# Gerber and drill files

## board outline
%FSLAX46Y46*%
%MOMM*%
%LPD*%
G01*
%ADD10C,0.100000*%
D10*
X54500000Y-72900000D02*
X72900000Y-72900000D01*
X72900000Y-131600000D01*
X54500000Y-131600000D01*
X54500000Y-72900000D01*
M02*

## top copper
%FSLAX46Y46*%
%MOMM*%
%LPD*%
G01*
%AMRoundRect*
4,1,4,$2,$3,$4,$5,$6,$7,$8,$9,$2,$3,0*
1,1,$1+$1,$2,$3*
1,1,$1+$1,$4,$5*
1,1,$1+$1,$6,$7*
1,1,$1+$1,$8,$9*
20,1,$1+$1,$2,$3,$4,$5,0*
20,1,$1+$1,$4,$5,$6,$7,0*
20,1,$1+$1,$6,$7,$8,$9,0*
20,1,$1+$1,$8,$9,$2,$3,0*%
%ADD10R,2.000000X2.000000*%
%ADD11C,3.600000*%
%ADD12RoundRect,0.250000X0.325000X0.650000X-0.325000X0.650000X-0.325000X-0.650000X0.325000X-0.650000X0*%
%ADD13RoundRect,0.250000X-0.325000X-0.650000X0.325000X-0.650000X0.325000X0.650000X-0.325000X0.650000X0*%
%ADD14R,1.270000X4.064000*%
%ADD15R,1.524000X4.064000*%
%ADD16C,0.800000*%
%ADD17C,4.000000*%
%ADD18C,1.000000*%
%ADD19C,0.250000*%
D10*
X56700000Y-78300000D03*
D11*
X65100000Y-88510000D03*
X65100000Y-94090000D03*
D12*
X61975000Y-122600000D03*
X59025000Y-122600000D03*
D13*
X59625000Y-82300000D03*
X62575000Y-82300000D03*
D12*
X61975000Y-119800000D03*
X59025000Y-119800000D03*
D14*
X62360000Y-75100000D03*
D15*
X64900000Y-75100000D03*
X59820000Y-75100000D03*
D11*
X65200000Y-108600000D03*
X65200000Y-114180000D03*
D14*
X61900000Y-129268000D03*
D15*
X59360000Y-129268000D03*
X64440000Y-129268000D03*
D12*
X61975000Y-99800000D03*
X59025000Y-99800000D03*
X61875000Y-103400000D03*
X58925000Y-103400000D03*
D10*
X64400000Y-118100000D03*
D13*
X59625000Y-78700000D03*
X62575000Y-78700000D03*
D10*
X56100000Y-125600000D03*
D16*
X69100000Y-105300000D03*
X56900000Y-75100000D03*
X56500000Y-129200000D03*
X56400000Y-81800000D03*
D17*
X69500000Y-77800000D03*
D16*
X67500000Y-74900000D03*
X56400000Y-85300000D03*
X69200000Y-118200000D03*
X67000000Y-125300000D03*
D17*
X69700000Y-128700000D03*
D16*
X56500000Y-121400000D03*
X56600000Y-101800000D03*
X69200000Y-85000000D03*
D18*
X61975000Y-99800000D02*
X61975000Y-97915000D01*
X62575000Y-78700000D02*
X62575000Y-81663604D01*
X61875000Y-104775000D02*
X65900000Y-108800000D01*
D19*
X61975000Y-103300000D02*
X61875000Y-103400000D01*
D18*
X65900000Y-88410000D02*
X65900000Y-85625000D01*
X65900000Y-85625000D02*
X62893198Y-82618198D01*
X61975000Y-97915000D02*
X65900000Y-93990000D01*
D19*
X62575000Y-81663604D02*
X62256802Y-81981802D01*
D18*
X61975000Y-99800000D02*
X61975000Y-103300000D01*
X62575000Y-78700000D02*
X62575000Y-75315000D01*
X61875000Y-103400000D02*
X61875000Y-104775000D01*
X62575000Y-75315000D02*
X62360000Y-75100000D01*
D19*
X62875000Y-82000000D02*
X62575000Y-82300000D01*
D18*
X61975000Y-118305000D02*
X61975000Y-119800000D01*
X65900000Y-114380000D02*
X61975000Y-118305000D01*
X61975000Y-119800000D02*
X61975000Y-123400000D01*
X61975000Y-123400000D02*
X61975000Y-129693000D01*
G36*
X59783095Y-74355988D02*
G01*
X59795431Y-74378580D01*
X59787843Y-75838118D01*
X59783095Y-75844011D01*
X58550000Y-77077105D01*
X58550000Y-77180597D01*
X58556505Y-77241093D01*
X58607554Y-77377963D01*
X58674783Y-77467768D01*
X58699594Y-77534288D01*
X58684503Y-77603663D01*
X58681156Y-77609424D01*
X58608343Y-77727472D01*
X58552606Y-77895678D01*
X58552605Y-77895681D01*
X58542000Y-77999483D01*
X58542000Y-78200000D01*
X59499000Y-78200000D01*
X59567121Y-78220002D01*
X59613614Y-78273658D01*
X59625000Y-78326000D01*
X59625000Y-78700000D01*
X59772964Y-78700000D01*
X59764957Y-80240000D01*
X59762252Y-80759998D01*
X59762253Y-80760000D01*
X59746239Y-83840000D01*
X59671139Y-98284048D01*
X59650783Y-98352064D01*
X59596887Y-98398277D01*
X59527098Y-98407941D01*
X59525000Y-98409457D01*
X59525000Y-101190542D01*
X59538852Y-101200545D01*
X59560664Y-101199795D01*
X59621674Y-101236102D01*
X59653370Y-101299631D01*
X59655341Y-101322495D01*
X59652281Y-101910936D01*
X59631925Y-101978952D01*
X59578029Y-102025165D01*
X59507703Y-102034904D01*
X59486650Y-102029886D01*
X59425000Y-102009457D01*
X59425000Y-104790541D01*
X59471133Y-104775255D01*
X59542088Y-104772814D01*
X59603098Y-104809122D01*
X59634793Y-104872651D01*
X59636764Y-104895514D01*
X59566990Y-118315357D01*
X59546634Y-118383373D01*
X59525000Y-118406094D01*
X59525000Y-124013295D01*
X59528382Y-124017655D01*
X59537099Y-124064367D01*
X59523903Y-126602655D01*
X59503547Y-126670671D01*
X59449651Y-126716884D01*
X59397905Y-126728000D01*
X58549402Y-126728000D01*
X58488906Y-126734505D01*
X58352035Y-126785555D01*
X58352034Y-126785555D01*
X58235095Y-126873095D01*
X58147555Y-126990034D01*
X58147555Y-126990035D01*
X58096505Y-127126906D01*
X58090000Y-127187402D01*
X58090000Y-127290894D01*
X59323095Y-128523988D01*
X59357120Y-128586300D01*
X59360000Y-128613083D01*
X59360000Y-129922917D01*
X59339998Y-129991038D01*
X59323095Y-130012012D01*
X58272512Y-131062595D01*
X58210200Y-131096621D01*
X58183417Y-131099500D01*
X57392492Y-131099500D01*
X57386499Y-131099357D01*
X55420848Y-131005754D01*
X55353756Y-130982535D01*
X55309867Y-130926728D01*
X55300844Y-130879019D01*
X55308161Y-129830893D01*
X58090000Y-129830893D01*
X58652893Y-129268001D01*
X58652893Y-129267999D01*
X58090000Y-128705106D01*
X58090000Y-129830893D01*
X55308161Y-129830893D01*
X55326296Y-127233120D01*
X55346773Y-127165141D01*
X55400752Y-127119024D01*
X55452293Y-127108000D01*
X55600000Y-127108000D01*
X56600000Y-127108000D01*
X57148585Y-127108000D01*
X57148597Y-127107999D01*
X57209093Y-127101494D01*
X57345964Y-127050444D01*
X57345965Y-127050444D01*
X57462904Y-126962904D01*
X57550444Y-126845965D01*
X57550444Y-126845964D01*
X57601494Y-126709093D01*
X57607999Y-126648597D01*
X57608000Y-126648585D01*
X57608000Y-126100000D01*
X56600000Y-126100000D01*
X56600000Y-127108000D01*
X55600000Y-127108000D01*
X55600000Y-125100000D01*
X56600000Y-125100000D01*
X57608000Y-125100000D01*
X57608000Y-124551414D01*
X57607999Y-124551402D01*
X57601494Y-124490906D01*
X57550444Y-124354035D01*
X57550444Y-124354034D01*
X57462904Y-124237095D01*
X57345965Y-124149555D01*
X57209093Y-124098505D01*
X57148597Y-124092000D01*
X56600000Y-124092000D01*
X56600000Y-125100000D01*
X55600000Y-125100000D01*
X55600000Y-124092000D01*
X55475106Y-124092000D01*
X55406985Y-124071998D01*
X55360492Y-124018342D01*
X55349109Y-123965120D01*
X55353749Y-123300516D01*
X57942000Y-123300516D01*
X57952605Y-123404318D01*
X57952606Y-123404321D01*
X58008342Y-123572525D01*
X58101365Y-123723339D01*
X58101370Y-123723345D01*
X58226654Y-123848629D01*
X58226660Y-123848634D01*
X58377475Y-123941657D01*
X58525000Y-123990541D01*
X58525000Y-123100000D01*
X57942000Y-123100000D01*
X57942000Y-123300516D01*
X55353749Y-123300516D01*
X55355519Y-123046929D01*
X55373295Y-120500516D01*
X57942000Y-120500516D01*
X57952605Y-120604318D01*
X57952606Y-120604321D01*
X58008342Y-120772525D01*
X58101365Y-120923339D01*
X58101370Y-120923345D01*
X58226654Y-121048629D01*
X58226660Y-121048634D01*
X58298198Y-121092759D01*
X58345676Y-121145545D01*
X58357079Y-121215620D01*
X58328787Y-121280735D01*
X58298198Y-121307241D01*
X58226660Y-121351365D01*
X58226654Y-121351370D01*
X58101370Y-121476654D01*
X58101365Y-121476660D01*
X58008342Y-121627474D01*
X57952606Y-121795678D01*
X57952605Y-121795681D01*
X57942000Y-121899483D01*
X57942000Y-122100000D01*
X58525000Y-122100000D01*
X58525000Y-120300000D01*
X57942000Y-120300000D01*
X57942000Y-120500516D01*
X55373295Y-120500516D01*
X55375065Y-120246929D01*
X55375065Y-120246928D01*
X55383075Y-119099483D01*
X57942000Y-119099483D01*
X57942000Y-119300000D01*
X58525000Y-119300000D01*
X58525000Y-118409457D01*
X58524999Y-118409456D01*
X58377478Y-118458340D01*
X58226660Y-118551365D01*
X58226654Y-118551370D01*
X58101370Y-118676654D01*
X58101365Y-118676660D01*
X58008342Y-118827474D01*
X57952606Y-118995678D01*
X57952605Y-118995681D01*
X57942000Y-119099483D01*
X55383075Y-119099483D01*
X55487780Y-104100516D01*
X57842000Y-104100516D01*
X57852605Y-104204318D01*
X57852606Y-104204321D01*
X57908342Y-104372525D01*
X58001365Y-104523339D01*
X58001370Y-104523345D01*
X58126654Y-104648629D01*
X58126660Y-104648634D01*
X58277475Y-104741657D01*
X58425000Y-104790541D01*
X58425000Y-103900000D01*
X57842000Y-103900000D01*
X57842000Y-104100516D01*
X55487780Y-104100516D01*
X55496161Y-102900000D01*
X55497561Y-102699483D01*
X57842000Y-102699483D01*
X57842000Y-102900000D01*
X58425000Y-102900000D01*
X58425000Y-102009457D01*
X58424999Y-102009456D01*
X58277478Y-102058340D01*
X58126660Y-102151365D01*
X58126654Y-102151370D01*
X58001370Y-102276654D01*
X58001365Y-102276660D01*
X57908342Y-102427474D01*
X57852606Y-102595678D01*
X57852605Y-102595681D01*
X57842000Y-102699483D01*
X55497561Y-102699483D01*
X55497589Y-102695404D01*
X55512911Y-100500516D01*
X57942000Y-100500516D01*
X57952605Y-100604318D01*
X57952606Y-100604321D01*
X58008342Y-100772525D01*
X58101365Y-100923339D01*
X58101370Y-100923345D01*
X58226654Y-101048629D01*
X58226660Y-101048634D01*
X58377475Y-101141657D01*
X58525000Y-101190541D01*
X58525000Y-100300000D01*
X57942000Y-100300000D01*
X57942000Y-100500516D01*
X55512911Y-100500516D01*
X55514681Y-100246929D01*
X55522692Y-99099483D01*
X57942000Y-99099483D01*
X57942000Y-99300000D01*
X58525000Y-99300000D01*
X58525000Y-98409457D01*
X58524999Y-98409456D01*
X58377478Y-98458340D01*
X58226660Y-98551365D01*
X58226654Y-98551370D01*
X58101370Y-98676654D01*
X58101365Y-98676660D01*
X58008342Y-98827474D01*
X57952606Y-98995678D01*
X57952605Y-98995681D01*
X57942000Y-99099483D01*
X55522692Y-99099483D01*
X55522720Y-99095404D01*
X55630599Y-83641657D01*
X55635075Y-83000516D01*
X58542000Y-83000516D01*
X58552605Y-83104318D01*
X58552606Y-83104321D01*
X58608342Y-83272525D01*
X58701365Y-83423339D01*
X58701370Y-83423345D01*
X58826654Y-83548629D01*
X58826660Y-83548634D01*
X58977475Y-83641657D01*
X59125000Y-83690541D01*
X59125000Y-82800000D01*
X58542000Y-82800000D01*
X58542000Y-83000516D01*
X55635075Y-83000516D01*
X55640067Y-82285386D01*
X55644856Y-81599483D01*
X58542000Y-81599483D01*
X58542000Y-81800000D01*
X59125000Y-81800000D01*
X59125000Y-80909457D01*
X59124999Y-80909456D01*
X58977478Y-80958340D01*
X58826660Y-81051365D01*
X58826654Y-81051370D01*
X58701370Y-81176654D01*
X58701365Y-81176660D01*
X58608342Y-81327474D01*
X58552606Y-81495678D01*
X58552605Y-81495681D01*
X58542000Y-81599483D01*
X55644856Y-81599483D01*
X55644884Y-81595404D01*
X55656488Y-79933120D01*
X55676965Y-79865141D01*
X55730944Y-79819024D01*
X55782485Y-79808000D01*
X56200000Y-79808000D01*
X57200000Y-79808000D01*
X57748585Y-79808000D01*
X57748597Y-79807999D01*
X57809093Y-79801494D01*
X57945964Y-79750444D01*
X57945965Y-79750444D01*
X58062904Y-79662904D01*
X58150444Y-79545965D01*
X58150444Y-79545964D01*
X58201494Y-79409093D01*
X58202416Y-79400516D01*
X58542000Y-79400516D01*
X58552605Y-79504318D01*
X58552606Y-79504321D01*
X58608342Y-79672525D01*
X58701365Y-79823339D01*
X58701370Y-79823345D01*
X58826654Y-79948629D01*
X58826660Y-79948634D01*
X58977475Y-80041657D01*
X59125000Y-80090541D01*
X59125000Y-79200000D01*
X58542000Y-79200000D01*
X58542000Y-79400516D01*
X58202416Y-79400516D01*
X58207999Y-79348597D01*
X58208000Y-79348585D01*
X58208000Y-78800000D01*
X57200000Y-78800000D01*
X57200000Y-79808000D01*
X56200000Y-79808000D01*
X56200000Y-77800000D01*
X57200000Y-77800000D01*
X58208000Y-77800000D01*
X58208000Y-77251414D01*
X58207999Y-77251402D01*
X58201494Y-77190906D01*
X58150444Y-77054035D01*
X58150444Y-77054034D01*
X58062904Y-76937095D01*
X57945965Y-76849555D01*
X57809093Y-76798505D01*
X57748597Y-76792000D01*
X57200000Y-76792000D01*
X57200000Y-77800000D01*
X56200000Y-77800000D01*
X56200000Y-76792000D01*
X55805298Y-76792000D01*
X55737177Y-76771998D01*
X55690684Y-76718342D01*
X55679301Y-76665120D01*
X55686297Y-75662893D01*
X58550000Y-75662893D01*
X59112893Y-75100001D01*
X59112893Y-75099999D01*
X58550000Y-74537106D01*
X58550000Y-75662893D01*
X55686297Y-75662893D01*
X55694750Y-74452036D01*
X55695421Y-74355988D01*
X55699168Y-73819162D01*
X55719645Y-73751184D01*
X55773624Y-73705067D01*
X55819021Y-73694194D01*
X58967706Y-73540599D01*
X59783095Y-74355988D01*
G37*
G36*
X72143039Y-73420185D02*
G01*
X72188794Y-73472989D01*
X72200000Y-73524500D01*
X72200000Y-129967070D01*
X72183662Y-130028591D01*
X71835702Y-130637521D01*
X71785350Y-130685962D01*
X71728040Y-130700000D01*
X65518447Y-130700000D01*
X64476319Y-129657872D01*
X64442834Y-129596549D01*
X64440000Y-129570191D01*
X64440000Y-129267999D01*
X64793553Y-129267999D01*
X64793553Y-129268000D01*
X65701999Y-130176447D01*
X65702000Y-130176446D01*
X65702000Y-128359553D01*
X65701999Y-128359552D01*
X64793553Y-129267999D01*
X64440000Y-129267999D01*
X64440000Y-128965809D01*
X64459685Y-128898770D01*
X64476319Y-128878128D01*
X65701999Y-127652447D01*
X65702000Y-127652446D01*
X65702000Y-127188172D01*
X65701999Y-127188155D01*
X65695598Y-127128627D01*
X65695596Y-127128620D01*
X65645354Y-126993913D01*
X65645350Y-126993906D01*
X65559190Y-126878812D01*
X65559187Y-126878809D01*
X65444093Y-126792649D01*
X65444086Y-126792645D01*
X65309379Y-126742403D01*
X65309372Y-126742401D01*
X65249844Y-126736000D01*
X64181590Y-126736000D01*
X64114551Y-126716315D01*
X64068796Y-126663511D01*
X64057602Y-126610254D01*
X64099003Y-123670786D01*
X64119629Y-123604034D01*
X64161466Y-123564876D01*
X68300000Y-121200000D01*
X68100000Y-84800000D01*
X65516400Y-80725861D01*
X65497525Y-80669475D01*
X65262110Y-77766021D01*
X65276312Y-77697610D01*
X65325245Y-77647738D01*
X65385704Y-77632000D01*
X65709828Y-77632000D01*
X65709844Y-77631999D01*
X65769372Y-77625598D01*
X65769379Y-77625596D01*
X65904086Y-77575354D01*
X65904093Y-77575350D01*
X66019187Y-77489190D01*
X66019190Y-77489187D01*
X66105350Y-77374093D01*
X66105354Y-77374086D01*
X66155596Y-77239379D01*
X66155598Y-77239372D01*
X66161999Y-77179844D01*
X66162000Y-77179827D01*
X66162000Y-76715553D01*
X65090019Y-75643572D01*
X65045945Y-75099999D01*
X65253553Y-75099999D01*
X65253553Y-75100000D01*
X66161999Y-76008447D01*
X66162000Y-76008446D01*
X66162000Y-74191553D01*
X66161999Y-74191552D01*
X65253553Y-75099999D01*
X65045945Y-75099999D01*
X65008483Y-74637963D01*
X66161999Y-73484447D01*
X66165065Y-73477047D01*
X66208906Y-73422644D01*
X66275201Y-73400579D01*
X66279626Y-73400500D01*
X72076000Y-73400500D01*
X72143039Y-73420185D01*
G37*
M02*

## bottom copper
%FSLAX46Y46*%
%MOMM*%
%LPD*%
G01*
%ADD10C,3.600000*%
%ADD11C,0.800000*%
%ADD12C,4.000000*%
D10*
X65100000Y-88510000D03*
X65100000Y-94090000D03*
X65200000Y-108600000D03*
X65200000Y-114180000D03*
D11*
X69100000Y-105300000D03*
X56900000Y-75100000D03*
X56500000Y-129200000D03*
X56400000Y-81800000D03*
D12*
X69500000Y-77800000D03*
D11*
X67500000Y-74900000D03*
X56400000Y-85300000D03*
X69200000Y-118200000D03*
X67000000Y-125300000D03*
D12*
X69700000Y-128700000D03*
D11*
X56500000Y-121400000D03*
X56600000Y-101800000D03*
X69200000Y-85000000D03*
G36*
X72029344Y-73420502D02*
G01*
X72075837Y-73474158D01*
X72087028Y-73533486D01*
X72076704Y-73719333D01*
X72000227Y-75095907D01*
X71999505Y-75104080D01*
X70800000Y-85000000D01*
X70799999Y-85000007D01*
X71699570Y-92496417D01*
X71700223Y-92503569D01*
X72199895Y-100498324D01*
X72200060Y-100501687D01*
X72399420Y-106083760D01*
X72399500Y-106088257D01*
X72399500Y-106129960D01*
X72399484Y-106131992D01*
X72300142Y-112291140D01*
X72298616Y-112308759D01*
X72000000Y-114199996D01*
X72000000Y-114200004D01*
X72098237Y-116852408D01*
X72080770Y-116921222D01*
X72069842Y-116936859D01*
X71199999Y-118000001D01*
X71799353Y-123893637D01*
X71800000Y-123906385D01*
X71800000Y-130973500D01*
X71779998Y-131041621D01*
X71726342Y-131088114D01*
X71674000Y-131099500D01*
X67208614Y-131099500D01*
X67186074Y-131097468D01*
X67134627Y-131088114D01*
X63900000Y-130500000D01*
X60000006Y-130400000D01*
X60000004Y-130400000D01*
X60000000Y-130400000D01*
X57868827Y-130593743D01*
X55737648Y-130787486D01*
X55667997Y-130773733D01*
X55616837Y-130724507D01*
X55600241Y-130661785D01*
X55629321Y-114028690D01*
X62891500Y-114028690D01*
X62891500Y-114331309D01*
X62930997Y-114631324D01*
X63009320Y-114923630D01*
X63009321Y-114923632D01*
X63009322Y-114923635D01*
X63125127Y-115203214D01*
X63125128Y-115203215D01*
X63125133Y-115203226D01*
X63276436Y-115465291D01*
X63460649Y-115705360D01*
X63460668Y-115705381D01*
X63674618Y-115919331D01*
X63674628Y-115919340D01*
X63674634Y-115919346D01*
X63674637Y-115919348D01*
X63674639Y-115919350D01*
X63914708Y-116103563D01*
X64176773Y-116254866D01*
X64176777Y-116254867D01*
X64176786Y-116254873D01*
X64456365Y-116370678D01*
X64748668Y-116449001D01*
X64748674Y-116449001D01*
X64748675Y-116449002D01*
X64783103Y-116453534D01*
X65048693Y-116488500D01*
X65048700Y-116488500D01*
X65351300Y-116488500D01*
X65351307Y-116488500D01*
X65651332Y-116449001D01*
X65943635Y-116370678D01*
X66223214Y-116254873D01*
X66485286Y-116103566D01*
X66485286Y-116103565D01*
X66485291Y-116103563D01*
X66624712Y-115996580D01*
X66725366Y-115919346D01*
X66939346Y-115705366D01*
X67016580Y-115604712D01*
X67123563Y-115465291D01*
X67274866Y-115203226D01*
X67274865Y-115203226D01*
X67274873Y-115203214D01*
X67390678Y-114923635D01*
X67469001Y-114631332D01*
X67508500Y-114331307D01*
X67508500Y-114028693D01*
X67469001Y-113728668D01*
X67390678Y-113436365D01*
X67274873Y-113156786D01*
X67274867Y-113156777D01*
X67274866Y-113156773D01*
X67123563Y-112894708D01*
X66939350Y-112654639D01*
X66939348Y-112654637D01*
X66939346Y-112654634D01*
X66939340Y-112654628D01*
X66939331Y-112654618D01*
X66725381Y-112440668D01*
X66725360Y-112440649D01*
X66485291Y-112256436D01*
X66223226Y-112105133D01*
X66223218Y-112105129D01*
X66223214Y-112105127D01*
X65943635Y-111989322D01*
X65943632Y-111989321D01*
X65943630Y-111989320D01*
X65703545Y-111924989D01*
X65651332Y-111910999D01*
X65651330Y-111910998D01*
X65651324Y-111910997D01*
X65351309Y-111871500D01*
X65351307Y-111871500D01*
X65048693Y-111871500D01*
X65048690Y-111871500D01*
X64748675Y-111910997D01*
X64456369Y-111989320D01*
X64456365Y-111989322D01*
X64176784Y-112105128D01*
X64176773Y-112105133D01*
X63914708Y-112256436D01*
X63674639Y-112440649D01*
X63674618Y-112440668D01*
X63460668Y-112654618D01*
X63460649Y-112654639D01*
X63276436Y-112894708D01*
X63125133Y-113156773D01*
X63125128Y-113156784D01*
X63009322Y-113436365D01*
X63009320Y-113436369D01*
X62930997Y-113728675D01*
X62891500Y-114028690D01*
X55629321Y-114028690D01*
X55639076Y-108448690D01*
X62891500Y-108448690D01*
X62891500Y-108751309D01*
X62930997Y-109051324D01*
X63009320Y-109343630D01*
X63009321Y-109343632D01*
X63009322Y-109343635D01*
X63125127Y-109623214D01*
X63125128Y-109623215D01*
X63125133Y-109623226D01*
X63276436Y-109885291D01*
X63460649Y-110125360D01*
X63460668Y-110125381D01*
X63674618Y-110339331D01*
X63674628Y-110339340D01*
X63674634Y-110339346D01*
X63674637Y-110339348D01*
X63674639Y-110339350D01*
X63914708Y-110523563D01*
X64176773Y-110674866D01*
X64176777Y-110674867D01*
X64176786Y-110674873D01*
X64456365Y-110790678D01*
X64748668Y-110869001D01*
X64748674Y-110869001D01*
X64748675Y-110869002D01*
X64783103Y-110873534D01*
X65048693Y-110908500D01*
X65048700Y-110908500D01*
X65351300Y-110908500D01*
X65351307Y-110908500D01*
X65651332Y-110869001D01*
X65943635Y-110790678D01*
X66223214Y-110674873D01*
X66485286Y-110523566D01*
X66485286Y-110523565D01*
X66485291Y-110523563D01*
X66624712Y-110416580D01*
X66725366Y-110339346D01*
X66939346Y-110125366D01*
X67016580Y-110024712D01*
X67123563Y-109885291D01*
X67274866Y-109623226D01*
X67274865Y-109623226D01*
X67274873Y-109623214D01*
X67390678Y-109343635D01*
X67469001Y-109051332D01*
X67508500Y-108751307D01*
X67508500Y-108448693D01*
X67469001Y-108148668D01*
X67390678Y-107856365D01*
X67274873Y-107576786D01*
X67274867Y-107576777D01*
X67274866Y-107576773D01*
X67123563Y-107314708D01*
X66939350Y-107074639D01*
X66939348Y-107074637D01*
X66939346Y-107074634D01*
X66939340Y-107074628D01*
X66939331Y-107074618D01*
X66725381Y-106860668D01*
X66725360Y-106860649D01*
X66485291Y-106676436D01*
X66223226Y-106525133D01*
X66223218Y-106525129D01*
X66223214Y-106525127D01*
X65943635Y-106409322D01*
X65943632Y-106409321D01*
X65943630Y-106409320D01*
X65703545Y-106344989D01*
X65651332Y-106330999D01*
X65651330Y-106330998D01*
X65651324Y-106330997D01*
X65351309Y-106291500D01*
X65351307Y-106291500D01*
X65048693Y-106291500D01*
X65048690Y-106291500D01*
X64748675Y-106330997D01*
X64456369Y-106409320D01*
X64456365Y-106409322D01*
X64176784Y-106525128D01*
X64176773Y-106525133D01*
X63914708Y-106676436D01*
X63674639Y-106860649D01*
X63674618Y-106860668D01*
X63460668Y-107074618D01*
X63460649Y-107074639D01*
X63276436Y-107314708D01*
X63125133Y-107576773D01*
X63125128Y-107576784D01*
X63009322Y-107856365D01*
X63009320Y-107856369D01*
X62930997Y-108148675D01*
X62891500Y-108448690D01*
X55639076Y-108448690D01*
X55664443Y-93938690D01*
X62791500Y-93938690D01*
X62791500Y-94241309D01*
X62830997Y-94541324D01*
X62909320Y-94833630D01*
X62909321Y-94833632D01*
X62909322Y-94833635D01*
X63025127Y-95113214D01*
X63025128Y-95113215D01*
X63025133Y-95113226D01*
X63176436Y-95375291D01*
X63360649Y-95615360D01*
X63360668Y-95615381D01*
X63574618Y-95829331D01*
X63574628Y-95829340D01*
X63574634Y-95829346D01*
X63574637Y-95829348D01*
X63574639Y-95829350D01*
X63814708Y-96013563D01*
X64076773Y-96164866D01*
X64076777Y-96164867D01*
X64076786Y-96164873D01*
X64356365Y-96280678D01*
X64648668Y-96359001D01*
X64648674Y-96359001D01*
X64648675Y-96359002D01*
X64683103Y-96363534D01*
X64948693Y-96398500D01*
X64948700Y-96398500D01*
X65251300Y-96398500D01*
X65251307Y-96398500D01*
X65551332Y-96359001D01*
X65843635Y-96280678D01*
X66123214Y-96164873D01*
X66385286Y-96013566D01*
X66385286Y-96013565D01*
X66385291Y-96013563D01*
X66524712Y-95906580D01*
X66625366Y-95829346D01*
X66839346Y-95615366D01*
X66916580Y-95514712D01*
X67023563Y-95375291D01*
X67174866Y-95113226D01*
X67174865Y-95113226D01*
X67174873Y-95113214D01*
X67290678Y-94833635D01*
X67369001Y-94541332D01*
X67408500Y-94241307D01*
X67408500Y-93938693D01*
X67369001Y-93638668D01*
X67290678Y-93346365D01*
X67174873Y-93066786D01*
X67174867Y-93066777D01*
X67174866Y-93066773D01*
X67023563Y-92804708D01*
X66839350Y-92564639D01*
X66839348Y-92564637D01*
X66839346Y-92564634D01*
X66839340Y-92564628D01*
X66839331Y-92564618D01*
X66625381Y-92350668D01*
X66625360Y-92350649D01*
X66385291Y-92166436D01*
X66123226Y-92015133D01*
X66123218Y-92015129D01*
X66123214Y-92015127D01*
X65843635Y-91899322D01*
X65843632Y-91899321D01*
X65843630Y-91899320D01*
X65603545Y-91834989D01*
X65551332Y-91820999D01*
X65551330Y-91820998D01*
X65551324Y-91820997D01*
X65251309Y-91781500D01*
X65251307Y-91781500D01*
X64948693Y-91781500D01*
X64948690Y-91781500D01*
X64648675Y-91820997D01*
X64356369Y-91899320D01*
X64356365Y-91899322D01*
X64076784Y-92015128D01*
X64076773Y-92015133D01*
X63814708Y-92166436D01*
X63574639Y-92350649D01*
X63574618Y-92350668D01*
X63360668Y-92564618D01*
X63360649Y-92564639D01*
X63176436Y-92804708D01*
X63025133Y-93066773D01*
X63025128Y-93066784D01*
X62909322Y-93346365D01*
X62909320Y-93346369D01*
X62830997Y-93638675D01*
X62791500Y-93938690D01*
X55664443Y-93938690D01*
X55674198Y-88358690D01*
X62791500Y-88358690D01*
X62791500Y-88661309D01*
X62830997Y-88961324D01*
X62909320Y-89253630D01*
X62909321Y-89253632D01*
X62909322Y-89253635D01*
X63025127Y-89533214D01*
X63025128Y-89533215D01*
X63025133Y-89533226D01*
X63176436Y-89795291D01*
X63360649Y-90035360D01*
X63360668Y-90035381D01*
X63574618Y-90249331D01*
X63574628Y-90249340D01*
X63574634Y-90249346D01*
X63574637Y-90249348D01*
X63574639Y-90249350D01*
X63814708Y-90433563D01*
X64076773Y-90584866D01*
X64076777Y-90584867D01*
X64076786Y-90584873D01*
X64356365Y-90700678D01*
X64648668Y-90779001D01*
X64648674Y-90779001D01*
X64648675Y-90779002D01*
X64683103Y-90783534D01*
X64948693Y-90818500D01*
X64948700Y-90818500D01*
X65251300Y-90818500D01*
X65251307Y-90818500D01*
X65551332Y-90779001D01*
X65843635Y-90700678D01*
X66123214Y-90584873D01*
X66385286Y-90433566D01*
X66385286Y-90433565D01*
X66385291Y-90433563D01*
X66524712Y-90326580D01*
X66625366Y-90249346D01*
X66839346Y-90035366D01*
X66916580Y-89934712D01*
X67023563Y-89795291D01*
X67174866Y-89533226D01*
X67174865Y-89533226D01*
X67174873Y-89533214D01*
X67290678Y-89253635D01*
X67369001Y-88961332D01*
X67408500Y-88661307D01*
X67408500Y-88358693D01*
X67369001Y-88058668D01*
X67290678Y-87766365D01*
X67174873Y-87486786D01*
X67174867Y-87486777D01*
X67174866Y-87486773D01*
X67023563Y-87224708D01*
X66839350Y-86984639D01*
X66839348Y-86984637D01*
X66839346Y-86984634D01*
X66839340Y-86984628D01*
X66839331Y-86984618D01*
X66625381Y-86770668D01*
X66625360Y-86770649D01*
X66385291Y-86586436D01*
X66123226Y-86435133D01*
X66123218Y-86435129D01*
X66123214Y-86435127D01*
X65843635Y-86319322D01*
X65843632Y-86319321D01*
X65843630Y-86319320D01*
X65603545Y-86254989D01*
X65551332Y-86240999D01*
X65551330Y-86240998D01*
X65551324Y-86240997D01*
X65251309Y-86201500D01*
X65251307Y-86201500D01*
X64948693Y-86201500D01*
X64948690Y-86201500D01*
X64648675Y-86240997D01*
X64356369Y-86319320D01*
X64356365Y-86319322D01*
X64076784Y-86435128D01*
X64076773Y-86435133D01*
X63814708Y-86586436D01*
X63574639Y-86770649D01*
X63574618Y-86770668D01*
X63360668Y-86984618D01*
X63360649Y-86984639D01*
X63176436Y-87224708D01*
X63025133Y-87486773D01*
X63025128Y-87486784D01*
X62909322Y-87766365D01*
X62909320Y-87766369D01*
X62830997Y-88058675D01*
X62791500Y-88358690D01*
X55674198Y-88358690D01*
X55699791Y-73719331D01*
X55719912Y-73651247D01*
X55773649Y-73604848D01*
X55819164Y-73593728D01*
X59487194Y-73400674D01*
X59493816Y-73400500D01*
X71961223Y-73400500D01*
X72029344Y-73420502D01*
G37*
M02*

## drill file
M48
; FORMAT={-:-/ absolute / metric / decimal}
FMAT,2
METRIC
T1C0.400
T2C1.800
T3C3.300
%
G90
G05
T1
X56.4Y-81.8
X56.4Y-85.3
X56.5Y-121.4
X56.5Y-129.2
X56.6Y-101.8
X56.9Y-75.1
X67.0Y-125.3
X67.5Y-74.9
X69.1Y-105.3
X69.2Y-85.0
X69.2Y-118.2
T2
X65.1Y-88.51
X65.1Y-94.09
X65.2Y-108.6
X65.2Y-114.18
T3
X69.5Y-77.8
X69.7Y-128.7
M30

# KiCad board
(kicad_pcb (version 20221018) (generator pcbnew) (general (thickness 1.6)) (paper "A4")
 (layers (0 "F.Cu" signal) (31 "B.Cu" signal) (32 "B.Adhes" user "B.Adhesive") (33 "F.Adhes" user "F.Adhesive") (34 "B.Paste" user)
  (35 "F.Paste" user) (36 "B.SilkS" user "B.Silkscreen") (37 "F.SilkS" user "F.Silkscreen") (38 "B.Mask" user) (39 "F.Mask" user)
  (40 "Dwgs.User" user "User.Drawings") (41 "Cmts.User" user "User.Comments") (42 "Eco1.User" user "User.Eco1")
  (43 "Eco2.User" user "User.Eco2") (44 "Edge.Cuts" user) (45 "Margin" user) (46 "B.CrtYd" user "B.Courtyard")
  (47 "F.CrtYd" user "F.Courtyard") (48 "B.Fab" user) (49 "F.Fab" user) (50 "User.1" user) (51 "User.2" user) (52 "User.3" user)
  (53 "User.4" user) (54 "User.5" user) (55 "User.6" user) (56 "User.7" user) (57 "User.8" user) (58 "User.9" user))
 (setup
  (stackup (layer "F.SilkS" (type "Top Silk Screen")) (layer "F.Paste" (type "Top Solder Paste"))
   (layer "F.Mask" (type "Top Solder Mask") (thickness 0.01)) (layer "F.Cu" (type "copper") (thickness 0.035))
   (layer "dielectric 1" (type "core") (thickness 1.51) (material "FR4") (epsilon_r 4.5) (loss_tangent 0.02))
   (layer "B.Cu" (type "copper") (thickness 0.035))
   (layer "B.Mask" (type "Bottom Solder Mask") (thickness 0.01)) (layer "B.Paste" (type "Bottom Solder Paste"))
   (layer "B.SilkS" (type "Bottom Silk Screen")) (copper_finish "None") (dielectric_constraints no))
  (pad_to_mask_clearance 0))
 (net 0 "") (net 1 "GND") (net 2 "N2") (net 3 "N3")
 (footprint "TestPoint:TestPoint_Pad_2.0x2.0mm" (layer "F.Cu") (at 56.7 78.3)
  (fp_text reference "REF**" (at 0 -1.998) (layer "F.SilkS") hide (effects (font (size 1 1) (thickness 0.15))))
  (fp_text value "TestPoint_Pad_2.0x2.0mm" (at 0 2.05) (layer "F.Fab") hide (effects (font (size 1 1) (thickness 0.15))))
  (pad "1" smd rect (at 0 0) (size 2 2) (layers "F.Cu" "F.Mask") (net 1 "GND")))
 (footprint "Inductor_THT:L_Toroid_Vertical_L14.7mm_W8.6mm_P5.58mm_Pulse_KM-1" (layer "F.Cu") (at 65.1 88.51)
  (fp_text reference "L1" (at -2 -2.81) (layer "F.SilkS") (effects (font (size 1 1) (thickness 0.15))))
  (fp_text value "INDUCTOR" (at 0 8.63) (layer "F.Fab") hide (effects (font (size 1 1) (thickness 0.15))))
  (pad "1" thru_hole circle (at 0 0) (size 3.6 3.6) (drill 1.8) (layers "*.Cu" "*.Mask") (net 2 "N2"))
  (pad "2" thru_hole circle (at 0 5.58) (size 3.6 3.6) (drill 1.8) (layers "*.Cu" "*.Mask") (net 2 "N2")))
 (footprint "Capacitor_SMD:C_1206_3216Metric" (layer "F.Cu") (at 60.5 122.6 180)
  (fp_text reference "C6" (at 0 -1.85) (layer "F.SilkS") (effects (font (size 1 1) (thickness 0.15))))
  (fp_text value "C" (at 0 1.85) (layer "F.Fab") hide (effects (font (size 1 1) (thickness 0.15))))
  (pad "1" smd roundrect (at -1.475 0 180) (size 1.15 1.8) (layers "F.Cu" "F.Paste" "F.Mask") (roundrect_rratio 0.2173913043) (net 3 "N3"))
  (pad "2" smd roundrect (at 1.475 0 180) (size 1.15 1.8) (layers "F.Cu" "F.Paste" "F.Mask") (roundrect_rratio 0.2173913043) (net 1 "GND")))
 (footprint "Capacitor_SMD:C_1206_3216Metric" (layer "F.Cu") (at 61.1 82.3)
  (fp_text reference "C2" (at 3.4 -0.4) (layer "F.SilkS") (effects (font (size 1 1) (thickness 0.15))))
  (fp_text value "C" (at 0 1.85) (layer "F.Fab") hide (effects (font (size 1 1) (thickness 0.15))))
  (pad "1" smd roundrect (at -1.475 0) (size 1.15 1.8) (layers "F.Cu" "F.Paste" "F.Mask") (roundrect_rratio 0.2173913043) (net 1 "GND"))
  (pad "2" smd roundrect (at 1.475 0) (size 1.15 1.8) (layers "F.Cu" "F.Paste" "F.Mask") (roundrect_rratio 0.2173913043) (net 2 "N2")))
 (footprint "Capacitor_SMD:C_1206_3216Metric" (layer "F.Cu") (at 60.5 119.8 180)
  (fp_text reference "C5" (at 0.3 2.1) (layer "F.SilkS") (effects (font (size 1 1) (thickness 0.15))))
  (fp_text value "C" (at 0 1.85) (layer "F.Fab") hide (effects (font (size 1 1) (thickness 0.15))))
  (pad "1" smd roundrect (at -1.475 0 180) (size 1.15 1.8) (layers "F.Cu" "F.Paste" "F.Mask") (roundrect_rratio 0.2173913043) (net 3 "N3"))
  (pad "2" smd roundrect (at 1.475 0 180) (size 1.15 1.8) (layers "F.Cu" "F.Paste" "F.Mask") (roundrect_rratio 0.2173913043) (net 1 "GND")))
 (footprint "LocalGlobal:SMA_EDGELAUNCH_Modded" (layer "F.Cu") (at 62.36 73.068 -90)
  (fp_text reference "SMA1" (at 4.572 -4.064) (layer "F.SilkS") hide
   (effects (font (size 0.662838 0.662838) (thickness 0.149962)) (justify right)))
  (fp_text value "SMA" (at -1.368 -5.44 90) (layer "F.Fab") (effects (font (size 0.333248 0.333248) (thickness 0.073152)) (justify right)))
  (pad "1" smd rect (at 2.032 0) (size 1.27 4.064) (layers "F.Cu" "F.Mask") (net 2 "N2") (solder_mask_margin 0.0508) (zone_connect 2)
   (thermal_bridge_angle 45))
  (pad "2" smd rect (at 2.032 -2.54) (size 1.524 4.064) (layers "F.Cu" "F.Mask") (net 1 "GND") (solder_mask_margin 0.0508)
   (thermal_bridge_angle 45))
  (pad "2" smd rect (at 2.032 2.54) (size 1.524 4.064) (layers "F.Cu" "F.Mask") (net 1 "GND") (solder_mask_margin 0.0508)
   (thermal_bridge_angle 45)))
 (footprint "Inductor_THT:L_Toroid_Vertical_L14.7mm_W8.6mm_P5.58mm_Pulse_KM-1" (layer "F.Cu") (at 65.2 108.6)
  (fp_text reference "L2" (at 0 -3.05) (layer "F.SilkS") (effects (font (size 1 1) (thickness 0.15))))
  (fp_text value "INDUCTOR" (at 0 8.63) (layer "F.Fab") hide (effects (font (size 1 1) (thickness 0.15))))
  (pad "1" thru_hole circle (at 0 0) (size 3.6 3.6) (drill 1.8) (layers "*.Cu" "*.Mask") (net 2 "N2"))
  (pad "2" thru_hole circle (at 0 5.58) (size 3.6 3.6) (drill 1.8) (layers "*.Cu" "*.Mask") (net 3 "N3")))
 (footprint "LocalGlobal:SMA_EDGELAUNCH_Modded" (layer "F.Cu") (at 61.9 131.3 90)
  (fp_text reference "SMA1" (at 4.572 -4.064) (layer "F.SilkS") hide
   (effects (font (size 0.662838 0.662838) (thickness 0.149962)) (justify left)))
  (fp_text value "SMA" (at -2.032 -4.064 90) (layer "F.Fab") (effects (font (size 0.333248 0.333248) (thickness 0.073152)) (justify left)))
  (pad "1" smd rect (at 2.032 0 180) (size 1.27 4.064) (layers "F.Cu" "F.Mask") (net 3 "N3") (solder_mask_margin 0.0508) (zone_connect 2)
   (thermal_bridge_angle 45))
  (pad "2" smd rect (at 2.032 -2.54 180) (size 1.524 4.064) (layers "F.Cu" "F.Mask") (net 1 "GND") (solder_mask_margin 0.0508)
   (thermal_bridge_angle 45))
  (pad "2" smd rect (at 2.032 2.54 180) (size 1.524 4.064) (layers "F.Cu" "F.Mask") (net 1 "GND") (solder_mask_margin 0.0508)
   (thermal_bridge_angle 45)))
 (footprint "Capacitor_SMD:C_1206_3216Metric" (layer "F.Cu") (at 60.5 99.8 180)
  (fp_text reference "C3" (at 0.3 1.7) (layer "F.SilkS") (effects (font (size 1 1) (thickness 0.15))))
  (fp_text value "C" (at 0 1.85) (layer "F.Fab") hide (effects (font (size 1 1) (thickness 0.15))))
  (pad "1" smd roundrect (at -1.475 0 180) (size 1.15 1.8) (layers "F.Cu" "F.Paste" "F.Mask") (roundrect_rratio 0.2173913043) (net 2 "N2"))
  (pad "2" smd roundrect (at 1.475 0 180) (size 1.15 1.8) (layers "F.Cu" "F.Paste" "F.Mask") (roundrect_rratio 0.2173913043) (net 1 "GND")))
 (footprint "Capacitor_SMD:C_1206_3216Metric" (layer "F.Cu") (at 60.4 103.4 180)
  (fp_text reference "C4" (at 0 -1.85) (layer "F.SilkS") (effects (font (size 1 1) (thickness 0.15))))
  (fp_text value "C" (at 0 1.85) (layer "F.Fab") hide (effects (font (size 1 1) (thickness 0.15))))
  (pad "1" smd roundrect (at -1.475 0 180) (size 1.15 1.8) (layers "F.Cu" "F.Paste" "F.Mask") (roundrect_rratio 0.2173913043) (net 2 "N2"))
  (pad "2" smd roundrect (at 1.475 0 180) (size 1.15 1.8) (layers "F.Cu" "F.Paste" "F.Mask") (roundrect_rratio 0.2173913043) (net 1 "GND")))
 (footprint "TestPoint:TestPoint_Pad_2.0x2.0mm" (layer "F.Cu") (at 64.4 118.1)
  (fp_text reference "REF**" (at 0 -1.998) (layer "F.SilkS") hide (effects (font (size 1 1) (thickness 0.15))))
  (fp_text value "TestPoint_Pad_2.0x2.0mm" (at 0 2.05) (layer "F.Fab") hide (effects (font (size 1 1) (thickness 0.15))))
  (pad "1" smd rect (at 0 0) (size 2 2) (layers "F.Cu" "F.Mask") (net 3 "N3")))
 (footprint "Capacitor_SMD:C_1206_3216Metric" (layer "F.Cu") (at 61.1 78.7)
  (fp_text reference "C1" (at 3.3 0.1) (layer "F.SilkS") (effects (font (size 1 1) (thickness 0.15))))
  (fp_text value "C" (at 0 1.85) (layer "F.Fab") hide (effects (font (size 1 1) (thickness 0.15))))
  (pad "1" smd roundrect (at -1.475 0) (size 1.15 1.8) (layers "F.Cu" "F.Paste" "F.Mask") (roundrect_rratio 0.2173913043) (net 1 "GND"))
  (pad "2" smd roundrect (at 1.475 0) (size 1.15 1.8) (layers "F.Cu" "F.Paste" "F.Mask") (roundrect_rratio 0.2173913043) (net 2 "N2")))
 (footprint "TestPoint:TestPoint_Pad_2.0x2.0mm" (layer "F.Cu") (at 56.1 125.6)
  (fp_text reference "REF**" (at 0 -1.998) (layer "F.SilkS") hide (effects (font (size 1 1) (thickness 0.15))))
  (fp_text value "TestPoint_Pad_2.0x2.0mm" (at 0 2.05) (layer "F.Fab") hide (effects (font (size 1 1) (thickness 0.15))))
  (pad "1" smd rect (at 0 0) (size 2 2) (layers "F.Cu" "F.Mask") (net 1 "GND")))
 (gr_rect (start 54.5 72.9) (end 72.9 131.6) (stroke (width 0.1) (type solid)) (fill none) (layer "Edge.Cuts"))
 (via (at 69.1 105.3) (size 0.8) (drill 0.4) (layers "F.Cu" "B.Cu") (free) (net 1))
 (via (at 56.9 75.1) (size 0.8) (drill 0.4) (layers "F.Cu" "B.Cu") (free) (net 1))
 (via (at 56.5 129.2) (size 0.8) (drill 0.4) (layers "F.Cu" "B.Cu") (free) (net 1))
 (via (at 56.4 81.8) (size 0.8) (drill 0.4) (layers "F.Cu" "B.Cu") (free) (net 1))
 (via (at 69.5 77.8) (size 4) (drill 3.3) (layers "F.Cu" "B.Cu") (free) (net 1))
 (via (at 67.5 74.9) (size 0.8) (drill 0.4) (layers "F.Cu" "B.Cu") (free) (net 1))
 (via (at 56.4 85.3) (size 0.8) (drill 0.4) (layers "F.Cu" "B.Cu") (free) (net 1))
 (via (at 69.2 118.2) (size 0.8) (drill 0.4) (layers "F.Cu" "B.Cu") (free) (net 1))
 (via (at 67 125.3) (size 0.8) (drill 0.4) (layers "F.Cu" "B.Cu") (free) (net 1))
 (via (at 69.7 128.7) (size 4) (drill 3.3) (layers "F.Cu" "B.Cu") (free) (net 1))
 (via (at 56.5 121.4) (size 0.8) (drill 0.4) (layers "F.Cu" "B.Cu") (free) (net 1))
 (via (at 56.6 101.8) (size 0.8) (drill 0.4) (layers "F.Cu" "B.Cu") (free) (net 1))
 (via (at 69.2 85) (size 0.8) (drill 0.4) (layers "F.Cu" "B.Cu") (free) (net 1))
 (segment (start 61.975 99.8) (end 61.975 97.915) (width 1) (layer "F.Cu") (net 2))
 (segment (start 62.575 78.7) (end 62.575 81.663604) (width 1) (layer "F.Cu") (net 2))
 (segment (start 61.875 104.775) (end 65.9 108.8) (width 1) (layer "F.Cu") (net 2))
 (segment (start 61.975 103.3) (end 61.875 103.4) (width 0.25) (layer "F.Cu") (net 2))
 (segment (start 65.9 88.41) (end 65.9 85.625) (width 1) (layer "F.Cu") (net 2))
 (segment (start 65.9 85.625) (end 62.893198 82.618198) (width 1) (layer "F.Cu") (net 2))
 (segment (start 61.975 97.915) (end 65.9 93.99) (width 1) (layer "F.Cu") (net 2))
 (segment (start 62.575 81.663604) (end 62.256802 81.981802) (width 0.25) (layer "F.Cu") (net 2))
 (segment (start 61.975 99.8) (end 61.975 103.3) (width 1) (layer "F.Cu") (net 2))
 (segment (start 62.575 78.7) (end 62.575 75.315) (width 1) (layer "F.Cu") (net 2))
 (segment (start 61.875 103.4) (end 61.875 104.775) (width 1) (layer "F.Cu") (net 2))
 (segment (start 62.575 75.315) (end 62.36 75.1) (width 1) (layer "F.Cu") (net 2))
 (segment (start 62.875 82) (end 62.575 82.3) (width 0.25) (layer "F.Cu") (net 2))
 (segment (start 61.975 118.305) (end 61.975 119.8) (width 1) (layer "F.Cu") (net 3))
 (segment (start 65.9 114.38) (end 61.975 118.305) (width 1) (layer "F.Cu") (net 3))
 (segment (start 61.975 119.8) (end 61.975 123.4) (width 1) (layer "F.Cu") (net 3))
 (segment (start 61.975 123.4) (end 61.975 129.693) (width 1) (layer "F.Cu") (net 3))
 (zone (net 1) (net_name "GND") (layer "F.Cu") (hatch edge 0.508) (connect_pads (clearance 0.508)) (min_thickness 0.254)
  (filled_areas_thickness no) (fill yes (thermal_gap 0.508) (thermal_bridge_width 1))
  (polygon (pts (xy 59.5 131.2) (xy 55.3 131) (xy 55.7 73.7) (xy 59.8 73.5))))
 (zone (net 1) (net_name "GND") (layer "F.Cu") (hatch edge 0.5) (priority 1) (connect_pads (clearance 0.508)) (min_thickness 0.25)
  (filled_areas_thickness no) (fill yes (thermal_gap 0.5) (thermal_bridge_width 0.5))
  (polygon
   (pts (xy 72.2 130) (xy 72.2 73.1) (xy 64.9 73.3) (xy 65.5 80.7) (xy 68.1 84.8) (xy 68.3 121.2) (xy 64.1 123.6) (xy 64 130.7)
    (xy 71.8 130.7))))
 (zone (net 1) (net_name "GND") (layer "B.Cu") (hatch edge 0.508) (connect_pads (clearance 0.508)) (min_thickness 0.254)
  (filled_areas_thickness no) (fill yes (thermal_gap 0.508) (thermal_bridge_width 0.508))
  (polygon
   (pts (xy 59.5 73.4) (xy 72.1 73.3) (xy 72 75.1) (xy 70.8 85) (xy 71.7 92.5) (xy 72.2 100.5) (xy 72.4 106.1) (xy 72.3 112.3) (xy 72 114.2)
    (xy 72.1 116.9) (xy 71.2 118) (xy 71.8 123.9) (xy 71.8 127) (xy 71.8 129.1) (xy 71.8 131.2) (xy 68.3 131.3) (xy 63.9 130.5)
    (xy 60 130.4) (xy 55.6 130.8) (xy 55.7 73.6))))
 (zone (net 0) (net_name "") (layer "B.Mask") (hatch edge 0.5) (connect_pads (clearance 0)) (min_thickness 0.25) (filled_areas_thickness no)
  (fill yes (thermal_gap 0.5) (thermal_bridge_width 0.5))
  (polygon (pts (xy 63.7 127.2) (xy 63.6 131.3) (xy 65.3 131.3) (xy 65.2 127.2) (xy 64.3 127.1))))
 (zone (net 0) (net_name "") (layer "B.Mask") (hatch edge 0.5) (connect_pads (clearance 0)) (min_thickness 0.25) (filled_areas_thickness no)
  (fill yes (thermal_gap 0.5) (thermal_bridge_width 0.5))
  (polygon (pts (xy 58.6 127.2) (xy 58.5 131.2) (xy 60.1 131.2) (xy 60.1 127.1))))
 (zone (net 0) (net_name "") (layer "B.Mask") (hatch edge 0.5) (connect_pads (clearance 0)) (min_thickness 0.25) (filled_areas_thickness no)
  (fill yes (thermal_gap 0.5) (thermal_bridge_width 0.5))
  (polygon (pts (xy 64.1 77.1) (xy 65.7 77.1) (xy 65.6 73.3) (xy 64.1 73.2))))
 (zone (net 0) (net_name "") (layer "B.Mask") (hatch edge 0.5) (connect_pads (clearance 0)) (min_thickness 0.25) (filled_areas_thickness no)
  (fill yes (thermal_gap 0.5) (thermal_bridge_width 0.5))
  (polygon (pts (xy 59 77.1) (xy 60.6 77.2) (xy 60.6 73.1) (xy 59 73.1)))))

